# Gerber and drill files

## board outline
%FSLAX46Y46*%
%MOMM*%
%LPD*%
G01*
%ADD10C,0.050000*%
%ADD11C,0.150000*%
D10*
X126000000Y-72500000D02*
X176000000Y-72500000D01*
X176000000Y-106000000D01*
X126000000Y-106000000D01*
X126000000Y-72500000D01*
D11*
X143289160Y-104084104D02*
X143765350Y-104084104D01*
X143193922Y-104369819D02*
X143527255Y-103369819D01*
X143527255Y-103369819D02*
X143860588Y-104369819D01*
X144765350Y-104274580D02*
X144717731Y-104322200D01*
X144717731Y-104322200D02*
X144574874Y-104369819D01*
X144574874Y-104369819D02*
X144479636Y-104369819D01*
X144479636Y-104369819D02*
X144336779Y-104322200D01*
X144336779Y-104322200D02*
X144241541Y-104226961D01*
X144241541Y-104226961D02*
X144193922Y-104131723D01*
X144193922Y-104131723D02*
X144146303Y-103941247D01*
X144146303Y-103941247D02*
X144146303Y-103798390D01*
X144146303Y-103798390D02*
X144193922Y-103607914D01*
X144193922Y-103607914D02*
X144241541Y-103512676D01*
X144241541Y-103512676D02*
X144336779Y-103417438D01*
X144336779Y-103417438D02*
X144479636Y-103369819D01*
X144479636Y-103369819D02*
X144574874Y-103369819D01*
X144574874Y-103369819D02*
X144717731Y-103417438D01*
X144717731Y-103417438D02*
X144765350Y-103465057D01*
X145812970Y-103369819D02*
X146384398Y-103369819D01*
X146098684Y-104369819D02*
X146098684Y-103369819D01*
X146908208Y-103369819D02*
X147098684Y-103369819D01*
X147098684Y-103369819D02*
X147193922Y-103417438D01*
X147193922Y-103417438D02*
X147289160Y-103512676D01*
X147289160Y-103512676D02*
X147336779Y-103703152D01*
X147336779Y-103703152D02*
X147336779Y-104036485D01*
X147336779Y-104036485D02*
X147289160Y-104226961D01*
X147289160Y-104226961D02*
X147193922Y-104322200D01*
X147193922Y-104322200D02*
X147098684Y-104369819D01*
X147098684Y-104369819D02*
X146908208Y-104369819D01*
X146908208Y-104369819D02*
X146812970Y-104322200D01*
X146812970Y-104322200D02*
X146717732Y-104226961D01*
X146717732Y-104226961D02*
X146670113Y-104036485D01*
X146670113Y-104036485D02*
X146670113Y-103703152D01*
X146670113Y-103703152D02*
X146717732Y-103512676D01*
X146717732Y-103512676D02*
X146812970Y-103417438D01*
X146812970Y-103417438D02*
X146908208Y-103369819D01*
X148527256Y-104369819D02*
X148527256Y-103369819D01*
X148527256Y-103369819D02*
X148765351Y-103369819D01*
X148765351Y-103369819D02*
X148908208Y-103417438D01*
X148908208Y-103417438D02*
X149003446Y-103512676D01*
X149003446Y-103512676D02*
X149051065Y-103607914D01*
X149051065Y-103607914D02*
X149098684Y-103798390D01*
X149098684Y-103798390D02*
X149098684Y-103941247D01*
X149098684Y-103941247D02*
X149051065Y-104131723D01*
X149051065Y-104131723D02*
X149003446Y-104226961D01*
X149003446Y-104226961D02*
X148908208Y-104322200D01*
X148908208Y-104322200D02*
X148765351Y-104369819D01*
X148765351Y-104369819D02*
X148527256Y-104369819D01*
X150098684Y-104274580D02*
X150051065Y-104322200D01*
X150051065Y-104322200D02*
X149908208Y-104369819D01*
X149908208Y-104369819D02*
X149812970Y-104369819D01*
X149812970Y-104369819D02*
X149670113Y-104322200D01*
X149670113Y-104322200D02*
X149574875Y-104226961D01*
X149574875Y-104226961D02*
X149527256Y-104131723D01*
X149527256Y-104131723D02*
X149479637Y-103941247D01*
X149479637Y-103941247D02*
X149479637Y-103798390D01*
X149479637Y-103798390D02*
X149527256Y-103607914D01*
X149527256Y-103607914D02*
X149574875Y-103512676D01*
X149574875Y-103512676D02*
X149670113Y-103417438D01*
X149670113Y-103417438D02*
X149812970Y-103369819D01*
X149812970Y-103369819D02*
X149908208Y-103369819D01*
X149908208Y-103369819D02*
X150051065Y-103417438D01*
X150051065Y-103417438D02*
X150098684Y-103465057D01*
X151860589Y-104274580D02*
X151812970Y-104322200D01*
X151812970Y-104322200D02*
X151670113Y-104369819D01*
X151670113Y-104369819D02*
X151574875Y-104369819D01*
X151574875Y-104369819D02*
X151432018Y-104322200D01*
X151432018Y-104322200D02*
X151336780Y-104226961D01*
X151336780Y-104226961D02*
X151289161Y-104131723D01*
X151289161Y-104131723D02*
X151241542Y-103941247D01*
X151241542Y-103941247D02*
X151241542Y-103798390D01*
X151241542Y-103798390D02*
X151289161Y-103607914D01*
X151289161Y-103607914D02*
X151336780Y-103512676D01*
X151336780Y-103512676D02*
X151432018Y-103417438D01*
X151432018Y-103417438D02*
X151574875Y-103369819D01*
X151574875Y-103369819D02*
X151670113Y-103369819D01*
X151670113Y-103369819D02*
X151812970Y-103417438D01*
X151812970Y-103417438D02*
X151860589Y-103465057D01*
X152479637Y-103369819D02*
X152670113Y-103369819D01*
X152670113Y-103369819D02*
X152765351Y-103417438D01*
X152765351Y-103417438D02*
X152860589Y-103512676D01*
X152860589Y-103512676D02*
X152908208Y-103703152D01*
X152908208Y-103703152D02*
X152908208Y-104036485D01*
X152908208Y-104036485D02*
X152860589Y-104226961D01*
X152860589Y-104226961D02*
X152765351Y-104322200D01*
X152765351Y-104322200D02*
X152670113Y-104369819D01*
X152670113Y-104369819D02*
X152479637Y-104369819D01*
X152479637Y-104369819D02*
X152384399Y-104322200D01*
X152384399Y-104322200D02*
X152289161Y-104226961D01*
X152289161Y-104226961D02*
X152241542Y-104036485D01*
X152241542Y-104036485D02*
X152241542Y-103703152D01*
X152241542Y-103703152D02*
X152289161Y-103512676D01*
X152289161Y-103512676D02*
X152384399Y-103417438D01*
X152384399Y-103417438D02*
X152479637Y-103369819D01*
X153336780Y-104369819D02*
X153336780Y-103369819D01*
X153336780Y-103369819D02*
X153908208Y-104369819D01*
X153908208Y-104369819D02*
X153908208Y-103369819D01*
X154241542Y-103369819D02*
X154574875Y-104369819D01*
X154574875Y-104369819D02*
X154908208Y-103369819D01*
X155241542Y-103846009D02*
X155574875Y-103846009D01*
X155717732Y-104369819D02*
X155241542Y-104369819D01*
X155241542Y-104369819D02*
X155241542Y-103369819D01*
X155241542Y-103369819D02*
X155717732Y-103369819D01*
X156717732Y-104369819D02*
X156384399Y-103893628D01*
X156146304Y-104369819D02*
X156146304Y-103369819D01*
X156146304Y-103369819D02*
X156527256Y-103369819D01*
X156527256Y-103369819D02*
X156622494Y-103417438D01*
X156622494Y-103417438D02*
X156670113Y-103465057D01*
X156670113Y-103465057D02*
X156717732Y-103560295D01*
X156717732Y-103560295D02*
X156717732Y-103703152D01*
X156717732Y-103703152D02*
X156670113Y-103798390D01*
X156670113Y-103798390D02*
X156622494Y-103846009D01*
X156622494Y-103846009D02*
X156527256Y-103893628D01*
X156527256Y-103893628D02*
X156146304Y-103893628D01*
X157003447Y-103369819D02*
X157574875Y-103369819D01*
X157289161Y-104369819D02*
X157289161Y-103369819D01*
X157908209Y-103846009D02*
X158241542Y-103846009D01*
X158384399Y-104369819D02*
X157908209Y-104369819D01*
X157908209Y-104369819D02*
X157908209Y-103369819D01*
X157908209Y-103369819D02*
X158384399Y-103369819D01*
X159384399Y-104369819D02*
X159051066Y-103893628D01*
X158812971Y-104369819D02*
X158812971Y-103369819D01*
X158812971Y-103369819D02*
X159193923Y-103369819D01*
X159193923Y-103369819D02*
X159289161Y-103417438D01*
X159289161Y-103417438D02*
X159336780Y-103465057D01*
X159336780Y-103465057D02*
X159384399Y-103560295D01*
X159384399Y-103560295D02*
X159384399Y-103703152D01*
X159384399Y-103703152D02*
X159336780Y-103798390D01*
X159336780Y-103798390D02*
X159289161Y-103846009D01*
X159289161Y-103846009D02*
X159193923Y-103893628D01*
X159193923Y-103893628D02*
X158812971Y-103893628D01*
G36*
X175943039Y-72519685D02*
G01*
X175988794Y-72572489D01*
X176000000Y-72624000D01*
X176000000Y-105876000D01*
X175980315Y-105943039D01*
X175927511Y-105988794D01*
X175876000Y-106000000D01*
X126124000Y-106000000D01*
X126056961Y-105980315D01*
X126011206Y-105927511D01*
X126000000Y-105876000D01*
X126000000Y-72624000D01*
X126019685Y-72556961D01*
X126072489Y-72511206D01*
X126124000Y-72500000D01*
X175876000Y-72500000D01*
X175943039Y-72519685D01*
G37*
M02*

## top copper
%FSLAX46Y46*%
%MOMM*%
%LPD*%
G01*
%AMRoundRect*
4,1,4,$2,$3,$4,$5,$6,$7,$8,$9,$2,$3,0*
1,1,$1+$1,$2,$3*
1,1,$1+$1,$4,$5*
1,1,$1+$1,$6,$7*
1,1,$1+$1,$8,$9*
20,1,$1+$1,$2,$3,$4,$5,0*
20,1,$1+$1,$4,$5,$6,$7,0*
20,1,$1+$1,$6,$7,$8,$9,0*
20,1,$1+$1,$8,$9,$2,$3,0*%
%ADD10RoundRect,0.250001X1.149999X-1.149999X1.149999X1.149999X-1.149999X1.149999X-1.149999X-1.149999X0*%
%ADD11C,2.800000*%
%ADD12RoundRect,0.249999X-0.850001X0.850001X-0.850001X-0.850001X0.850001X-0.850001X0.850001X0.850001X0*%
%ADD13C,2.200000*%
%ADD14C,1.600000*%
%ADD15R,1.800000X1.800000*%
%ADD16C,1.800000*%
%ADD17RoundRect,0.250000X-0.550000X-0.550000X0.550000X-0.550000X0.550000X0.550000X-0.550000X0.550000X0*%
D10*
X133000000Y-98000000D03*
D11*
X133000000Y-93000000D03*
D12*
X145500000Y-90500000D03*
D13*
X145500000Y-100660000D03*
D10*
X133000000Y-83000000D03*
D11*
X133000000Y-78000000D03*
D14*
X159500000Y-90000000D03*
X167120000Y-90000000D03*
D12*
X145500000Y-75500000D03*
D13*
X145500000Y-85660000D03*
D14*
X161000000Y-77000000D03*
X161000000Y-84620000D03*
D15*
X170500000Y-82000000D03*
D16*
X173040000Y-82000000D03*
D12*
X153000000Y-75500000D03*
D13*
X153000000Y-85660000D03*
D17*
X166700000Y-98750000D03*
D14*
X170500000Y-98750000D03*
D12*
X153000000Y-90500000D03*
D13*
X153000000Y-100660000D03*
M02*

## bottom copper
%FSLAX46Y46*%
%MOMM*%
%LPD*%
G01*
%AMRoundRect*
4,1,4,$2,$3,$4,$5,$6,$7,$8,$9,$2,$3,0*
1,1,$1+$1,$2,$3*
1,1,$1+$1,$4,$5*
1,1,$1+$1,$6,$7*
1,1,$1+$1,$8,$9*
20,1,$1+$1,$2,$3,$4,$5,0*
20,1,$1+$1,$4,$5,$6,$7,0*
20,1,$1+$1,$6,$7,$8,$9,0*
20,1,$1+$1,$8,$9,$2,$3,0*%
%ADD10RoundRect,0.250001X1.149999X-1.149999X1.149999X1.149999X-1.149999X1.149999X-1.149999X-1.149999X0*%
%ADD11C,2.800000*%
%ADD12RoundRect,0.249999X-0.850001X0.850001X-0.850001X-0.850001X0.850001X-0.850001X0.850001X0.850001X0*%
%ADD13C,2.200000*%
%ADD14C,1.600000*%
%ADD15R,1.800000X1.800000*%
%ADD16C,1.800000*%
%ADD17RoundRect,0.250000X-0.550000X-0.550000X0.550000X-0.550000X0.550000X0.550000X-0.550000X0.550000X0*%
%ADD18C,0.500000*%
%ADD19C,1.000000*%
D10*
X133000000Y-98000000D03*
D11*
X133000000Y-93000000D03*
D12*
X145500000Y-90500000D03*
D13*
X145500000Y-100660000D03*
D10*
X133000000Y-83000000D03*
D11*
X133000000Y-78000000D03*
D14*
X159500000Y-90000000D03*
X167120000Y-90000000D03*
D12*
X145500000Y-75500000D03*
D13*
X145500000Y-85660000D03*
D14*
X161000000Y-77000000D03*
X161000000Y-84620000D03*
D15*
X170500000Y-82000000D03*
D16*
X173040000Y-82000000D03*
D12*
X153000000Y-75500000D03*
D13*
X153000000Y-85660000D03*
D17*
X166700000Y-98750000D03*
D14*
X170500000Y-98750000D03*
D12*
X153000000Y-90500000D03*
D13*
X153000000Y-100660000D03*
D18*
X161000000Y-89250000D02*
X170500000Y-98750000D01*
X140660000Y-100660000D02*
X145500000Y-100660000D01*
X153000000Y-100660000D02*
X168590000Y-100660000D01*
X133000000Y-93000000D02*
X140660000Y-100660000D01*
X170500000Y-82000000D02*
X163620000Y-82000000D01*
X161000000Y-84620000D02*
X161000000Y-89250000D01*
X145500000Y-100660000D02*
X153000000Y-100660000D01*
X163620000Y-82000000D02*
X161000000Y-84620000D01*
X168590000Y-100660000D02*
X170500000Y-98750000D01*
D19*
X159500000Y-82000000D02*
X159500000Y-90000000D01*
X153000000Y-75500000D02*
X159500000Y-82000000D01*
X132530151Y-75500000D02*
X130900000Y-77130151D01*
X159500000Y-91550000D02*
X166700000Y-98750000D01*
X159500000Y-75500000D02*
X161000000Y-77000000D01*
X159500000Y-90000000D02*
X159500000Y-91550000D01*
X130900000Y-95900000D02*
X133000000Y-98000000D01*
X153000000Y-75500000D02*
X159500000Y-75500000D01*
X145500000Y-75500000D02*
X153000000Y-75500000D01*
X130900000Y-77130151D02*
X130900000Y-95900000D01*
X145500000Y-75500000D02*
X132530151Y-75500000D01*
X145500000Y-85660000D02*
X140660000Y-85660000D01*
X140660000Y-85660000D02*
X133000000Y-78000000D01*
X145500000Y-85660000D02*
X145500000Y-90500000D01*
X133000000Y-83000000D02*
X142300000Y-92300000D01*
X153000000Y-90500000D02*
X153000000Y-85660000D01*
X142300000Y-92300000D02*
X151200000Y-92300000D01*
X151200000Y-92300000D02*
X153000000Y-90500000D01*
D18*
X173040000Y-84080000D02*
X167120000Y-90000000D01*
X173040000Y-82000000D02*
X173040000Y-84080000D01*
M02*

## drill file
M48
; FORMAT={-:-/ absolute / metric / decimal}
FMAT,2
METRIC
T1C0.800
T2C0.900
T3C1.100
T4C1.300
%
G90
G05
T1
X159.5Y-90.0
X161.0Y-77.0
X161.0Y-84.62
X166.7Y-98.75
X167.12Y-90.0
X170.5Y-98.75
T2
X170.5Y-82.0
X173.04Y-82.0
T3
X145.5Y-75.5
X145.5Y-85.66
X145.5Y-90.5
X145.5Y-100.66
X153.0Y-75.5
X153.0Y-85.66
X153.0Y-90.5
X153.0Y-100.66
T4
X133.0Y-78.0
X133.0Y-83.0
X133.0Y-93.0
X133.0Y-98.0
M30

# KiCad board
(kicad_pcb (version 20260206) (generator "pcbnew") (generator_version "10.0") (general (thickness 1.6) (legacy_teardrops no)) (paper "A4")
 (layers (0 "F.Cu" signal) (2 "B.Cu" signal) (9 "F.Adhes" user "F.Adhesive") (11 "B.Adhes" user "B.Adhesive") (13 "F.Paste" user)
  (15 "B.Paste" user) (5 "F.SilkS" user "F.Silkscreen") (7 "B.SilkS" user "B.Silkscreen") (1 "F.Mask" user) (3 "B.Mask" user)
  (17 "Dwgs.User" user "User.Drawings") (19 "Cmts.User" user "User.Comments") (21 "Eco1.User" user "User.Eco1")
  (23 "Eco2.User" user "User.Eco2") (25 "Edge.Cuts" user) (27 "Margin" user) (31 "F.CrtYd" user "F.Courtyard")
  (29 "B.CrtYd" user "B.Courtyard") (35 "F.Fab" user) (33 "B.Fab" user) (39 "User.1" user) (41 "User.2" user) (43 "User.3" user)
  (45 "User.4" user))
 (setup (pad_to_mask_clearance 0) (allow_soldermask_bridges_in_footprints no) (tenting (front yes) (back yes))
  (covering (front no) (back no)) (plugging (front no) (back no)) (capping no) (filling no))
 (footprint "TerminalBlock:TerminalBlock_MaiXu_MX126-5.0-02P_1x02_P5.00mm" (layer "F.Cu") (at 133 98 90)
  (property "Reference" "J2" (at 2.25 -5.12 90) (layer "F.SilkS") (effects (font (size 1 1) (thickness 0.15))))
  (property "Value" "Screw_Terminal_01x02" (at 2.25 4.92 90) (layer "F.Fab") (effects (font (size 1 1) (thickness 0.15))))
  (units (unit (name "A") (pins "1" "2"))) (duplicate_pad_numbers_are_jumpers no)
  (pad "1" thru_hole roundrect (at 0 0 90) (size 2.8 2.8) (drill 1.3) (layers "*.Cu" "*.Mask") (remove_unused_layers no)
   (roundrect_rratio 0.089286) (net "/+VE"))
  (pad "2" thru_hole circle (at 5 0 90) (size 2.8 2.8) (drill 1.3) (layers "*.Cu" "*.Mask") (remove_unused_layers no) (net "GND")))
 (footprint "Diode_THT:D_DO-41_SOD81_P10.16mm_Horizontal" (layer "F.Cu") (at 145.5 90.5 -90)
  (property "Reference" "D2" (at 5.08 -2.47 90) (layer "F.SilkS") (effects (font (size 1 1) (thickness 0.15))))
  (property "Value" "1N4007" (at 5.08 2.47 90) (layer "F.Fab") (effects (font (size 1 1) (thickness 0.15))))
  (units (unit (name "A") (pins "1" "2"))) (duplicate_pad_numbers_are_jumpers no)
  (pad "1" thru_hole roundrect (at 0 0 270) (size 2.2 2.2) (drill 1.1) (layers "*.Cu" "*.Mask") (remove_unused_layers no)
   (roundrect_rratio 0.113636) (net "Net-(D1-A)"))
  (pad "2" thru_hole circle (at 10.16 0 270) (size 2.2 2.2) (drill 1.1) (layers "*.Cu" "*.Mask") (remove_unused_layers no) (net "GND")))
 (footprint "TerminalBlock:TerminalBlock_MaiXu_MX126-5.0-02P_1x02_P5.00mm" (layer "F.Cu") (at 133 83 90)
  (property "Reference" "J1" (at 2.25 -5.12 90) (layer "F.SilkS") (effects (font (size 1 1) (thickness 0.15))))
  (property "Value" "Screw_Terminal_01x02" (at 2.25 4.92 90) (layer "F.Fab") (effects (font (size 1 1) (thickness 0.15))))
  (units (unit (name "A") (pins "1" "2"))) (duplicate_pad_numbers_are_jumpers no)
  (pad "1" thru_hole roundrect (at 0 0 90) (size 2.8 2.8) (drill 1.3) (layers "*.Cu" "*.Mask") (remove_unused_layers no)
   (roundrect_rratio 0.089286) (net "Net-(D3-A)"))
  (pad "2" thru_hole circle (at 5 0 90) (size 2.8 2.8) (drill 1.3) (layers "*.Cu" "*.Mask") (remove_unused_layers no) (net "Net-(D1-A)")))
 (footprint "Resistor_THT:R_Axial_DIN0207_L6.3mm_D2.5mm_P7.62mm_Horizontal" (layer "F.Cu") (at 159.5 90)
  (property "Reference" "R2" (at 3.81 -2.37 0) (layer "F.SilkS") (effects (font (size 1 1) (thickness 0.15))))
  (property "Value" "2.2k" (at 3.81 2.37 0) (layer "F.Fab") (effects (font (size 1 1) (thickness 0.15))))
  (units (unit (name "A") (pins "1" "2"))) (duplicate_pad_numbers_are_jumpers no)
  (pad "1" thru_hole circle (at 0 0) (size 1.6 1.6) (drill 0.8) (layers "*.Cu" "*.Mask") (remove_unused_layers no) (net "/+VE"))
  (pad "2" thru_hole circle (at 7.62 0) (size 1.6 1.6) (drill 0.8) (layers "*.Cu" "*.Mask") (remove_unused_layers no) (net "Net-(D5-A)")))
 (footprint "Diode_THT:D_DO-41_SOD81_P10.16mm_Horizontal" (layer "F.Cu") (at 145.5 75.5 -90)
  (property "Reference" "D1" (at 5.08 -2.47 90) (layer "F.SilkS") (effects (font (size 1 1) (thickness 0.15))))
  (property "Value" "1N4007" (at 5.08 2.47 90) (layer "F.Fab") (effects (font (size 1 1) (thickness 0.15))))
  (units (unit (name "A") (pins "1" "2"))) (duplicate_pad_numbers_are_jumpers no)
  (pad "1" thru_hole roundrect (at 0 0 270) (size 2.2 2.2) (drill 1.1) (layers "*.Cu" "*.Mask") (remove_unused_layers no)
   (roundrect_rratio 0.113636) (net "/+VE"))
  (pad "2" thru_hole circle (at 10.16 0 270) (size 2.2 2.2) (drill 1.1) (layers "*.Cu" "*.Mask") (remove_unused_layers no)
   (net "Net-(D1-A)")))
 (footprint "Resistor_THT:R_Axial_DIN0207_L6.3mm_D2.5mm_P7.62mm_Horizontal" (layer "F.Cu") (at 161 77 -90)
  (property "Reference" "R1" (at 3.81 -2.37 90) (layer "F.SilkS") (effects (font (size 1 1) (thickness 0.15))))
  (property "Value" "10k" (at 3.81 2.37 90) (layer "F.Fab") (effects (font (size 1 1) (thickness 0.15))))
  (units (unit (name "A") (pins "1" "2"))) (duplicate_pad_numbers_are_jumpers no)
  (pad "1" thru_hole circle (at 0 0 270) (size 1.6 1.6) (drill 0.8) (layers "*.Cu" "*.Mask") (remove_unused_layers no) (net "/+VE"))
  (pad "2" thru_hole circle (at 7.62 0 270) (size 1.6 1.6) (drill 0.8) (layers "*.Cu" "*.Mask") (remove_unused_layers no) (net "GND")))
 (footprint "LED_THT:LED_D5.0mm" (layer "F.Cu") (at 170.5 82)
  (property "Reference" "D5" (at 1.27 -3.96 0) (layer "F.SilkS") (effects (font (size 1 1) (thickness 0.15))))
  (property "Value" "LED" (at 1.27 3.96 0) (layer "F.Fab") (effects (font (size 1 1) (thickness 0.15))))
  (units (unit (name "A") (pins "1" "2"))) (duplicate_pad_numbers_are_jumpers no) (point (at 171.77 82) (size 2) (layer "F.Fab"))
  (pad "1" thru_hole rect (at 0 0) (size 1.8 1.8) (drill 0.9) (layers "*.Cu" "*.Mask") (remove_unused_layers no) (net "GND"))
  (pad "2" thru_hole circle (at 2.54 0) (size 1.8 1.8) (drill 0.9) (layers "*.Cu" "*.Mask") (remove_unused_layers no) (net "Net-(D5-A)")))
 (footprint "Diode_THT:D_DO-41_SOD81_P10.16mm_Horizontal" (layer "F.Cu") (at 153 75.5 -90)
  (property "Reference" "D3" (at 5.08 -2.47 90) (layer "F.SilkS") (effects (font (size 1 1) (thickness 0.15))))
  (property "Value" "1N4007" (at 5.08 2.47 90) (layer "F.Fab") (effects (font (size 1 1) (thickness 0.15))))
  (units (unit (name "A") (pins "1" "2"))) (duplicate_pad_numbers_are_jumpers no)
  (pad "1" thru_hole roundrect (at 0 0 270) (size 2.2 2.2) (drill 1.1) (layers "*.Cu" "*.Mask") (remove_unused_layers no)
   (roundrect_rratio 0.113636) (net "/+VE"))
  (pad "2" thru_hole circle (at 10.16 0 270) (size 2.2 2.2) (drill 1.1) (layers "*.Cu" "*.Mask") (remove_unused_layers no)
   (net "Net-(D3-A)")))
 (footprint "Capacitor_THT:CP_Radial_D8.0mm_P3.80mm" (layer "F.Cu") (at 166.7 98.75)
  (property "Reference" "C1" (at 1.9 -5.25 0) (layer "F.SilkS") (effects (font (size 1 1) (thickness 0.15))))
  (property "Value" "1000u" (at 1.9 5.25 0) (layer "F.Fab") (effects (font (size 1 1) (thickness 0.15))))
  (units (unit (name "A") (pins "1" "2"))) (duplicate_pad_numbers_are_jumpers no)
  (pad "1" thru_hole roundrect (at 0 0) (size 1.6 1.6) (drill 0.8) (layers "*.Cu" "*.Mask") (remove_unused_layers no)
   (roundrect_rratio 0.15625) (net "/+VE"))
  (pad "2" thru_hole circle (at 3.8 0) (size 1.6 1.6) (drill 0.8) (layers "*.Cu" "*.Mask") (remove_unused_layers no) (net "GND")))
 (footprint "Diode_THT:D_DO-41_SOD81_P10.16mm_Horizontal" (layer "F.Cu") (at 153 90.5 -90)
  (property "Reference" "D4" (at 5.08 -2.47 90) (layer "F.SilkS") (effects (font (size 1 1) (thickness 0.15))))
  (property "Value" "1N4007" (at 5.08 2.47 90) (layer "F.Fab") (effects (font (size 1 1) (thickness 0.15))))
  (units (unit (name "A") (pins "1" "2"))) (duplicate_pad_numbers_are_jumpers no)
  (pad "1" thru_hole roundrect (at 0 0 270) (size 2.2 2.2) (drill 1.1) (layers "*.Cu" "*.Mask") (remove_unused_layers no)
   (roundrect_rratio 0.113636) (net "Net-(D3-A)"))
  (pad "2" thru_hole circle (at 10.16 0 270) (size 2.2 2.2) (drill 1.1) (layers "*.Cu" "*.Mask") (remove_unused_layers no) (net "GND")))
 (gr_rect (start 126 72.5) (end 176 106) (stroke (width 0.05) (type default)) (fill no) (layer "Edge.Cuts"))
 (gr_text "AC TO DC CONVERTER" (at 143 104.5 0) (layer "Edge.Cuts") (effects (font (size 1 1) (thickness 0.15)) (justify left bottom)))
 (segment (start 161 89.25) (end 170.5 98.75) (width 0.5) (layer "B.Cu") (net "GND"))
 (segment (start 140.66 100.66) (end 145.5 100.66) (width 0.5) (layer "B.Cu") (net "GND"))
 (segment (start 153 100.66) (end 168.59 100.66) (width 0.5) (layer "B.Cu") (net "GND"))
 (segment (start 133 93) (end 140.66 100.66) (width 0.5) (layer "B.Cu") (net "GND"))
 (segment (start 170.5 82) (end 163.62 82) (width 0.5) (layer "B.Cu") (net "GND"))
 (segment (start 161 84.62) (end 161 89.25) (width 0.5) (layer "B.Cu") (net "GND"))
 (segment (start 145.5 100.66) (end 153 100.66) (width 0.5) (layer "B.Cu") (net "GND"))
 (segment (start 163.62 82) (end 161 84.62) (width 0.5) (layer "B.Cu") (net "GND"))
 (segment (start 168.59 100.66) (end 170.5 98.75) (width 0.5) (layer "B.Cu") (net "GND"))
 (segment (start 159.5 82) (end 159.5 90) (width 1) (layer "B.Cu") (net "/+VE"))
 (segment (start 153 75.5) (end 159.5 82) (width 1) (layer "B.Cu") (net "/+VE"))
 (segment (start 132.530151 75.5) (end 130.9 77.130151) (width 1) (layer "B.Cu") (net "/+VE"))
 (segment (start 159.5 91.55) (end 166.7 98.75) (width 1) (layer "B.Cu") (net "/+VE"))
 (segment (start 159.5 75.5) (end 161 77) (width 1) (layer "B.Cu") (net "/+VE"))
 (segment (start 159.5 90) (end 159.5 91.55) (width 1) (layer "B.Cu") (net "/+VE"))
 (segment (start 130.9 95.9) (end 133 98) (width 1) (layer "B.Cu") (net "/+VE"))
 (segment (start 153 75.5) (end 159.5 75.5) (width 1) (layer "B.Cu") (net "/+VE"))
 (segment (start 145.5 75.5) (end 153 75.5) (width 1) (layer "B.Cu") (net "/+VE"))
 (segment (start 130.9 77.130151) (end 130.9 95.9) (width 1) (layer "B.Cu") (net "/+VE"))
 (segment (start 145.5 75.5) (end 132.530151 75.5) (width 1) (layer "B.Cu") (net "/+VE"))
 (segment (start 145.5 85.66) (end 140.66 85.66) (width 1) (layer "B.Cu") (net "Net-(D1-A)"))
 (segment (start 140.66 85.66) (end 133 78) (width 1) (layer "B.Cu") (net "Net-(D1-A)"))
 (segment (start 145.5 85.66) (end 145.5 90.5) (width 1) (layer "B.Cu") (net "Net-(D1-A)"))
 (segment (start 133 83) (end 142.3 92.3) (width 1) (layer "B.Cu") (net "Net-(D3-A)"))
 (segment (start 153 90.5) (end 153 85.66) (width 1) (layer "B.Cu") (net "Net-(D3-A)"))
 (segment (start 142.3 92.3) (end 151.2 92.3) (width 1) (layer "B.Cu") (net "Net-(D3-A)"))
 (segment (start 151.2 92.3) (end 153 90.5) (width 1) (layer "B.Cu") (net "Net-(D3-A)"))
 (segment (start 173.04 84.08) (end 167.12 90) (width 0.5) (layer "B.Cu") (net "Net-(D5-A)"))
 (segment (start 173.04 82) (end 173.04 84.08) (width 0.5) (layer "B.Cu") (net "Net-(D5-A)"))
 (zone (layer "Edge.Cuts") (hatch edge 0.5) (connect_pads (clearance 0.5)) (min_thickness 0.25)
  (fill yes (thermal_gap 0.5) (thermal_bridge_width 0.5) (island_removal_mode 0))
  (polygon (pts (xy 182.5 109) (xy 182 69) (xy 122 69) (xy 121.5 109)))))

